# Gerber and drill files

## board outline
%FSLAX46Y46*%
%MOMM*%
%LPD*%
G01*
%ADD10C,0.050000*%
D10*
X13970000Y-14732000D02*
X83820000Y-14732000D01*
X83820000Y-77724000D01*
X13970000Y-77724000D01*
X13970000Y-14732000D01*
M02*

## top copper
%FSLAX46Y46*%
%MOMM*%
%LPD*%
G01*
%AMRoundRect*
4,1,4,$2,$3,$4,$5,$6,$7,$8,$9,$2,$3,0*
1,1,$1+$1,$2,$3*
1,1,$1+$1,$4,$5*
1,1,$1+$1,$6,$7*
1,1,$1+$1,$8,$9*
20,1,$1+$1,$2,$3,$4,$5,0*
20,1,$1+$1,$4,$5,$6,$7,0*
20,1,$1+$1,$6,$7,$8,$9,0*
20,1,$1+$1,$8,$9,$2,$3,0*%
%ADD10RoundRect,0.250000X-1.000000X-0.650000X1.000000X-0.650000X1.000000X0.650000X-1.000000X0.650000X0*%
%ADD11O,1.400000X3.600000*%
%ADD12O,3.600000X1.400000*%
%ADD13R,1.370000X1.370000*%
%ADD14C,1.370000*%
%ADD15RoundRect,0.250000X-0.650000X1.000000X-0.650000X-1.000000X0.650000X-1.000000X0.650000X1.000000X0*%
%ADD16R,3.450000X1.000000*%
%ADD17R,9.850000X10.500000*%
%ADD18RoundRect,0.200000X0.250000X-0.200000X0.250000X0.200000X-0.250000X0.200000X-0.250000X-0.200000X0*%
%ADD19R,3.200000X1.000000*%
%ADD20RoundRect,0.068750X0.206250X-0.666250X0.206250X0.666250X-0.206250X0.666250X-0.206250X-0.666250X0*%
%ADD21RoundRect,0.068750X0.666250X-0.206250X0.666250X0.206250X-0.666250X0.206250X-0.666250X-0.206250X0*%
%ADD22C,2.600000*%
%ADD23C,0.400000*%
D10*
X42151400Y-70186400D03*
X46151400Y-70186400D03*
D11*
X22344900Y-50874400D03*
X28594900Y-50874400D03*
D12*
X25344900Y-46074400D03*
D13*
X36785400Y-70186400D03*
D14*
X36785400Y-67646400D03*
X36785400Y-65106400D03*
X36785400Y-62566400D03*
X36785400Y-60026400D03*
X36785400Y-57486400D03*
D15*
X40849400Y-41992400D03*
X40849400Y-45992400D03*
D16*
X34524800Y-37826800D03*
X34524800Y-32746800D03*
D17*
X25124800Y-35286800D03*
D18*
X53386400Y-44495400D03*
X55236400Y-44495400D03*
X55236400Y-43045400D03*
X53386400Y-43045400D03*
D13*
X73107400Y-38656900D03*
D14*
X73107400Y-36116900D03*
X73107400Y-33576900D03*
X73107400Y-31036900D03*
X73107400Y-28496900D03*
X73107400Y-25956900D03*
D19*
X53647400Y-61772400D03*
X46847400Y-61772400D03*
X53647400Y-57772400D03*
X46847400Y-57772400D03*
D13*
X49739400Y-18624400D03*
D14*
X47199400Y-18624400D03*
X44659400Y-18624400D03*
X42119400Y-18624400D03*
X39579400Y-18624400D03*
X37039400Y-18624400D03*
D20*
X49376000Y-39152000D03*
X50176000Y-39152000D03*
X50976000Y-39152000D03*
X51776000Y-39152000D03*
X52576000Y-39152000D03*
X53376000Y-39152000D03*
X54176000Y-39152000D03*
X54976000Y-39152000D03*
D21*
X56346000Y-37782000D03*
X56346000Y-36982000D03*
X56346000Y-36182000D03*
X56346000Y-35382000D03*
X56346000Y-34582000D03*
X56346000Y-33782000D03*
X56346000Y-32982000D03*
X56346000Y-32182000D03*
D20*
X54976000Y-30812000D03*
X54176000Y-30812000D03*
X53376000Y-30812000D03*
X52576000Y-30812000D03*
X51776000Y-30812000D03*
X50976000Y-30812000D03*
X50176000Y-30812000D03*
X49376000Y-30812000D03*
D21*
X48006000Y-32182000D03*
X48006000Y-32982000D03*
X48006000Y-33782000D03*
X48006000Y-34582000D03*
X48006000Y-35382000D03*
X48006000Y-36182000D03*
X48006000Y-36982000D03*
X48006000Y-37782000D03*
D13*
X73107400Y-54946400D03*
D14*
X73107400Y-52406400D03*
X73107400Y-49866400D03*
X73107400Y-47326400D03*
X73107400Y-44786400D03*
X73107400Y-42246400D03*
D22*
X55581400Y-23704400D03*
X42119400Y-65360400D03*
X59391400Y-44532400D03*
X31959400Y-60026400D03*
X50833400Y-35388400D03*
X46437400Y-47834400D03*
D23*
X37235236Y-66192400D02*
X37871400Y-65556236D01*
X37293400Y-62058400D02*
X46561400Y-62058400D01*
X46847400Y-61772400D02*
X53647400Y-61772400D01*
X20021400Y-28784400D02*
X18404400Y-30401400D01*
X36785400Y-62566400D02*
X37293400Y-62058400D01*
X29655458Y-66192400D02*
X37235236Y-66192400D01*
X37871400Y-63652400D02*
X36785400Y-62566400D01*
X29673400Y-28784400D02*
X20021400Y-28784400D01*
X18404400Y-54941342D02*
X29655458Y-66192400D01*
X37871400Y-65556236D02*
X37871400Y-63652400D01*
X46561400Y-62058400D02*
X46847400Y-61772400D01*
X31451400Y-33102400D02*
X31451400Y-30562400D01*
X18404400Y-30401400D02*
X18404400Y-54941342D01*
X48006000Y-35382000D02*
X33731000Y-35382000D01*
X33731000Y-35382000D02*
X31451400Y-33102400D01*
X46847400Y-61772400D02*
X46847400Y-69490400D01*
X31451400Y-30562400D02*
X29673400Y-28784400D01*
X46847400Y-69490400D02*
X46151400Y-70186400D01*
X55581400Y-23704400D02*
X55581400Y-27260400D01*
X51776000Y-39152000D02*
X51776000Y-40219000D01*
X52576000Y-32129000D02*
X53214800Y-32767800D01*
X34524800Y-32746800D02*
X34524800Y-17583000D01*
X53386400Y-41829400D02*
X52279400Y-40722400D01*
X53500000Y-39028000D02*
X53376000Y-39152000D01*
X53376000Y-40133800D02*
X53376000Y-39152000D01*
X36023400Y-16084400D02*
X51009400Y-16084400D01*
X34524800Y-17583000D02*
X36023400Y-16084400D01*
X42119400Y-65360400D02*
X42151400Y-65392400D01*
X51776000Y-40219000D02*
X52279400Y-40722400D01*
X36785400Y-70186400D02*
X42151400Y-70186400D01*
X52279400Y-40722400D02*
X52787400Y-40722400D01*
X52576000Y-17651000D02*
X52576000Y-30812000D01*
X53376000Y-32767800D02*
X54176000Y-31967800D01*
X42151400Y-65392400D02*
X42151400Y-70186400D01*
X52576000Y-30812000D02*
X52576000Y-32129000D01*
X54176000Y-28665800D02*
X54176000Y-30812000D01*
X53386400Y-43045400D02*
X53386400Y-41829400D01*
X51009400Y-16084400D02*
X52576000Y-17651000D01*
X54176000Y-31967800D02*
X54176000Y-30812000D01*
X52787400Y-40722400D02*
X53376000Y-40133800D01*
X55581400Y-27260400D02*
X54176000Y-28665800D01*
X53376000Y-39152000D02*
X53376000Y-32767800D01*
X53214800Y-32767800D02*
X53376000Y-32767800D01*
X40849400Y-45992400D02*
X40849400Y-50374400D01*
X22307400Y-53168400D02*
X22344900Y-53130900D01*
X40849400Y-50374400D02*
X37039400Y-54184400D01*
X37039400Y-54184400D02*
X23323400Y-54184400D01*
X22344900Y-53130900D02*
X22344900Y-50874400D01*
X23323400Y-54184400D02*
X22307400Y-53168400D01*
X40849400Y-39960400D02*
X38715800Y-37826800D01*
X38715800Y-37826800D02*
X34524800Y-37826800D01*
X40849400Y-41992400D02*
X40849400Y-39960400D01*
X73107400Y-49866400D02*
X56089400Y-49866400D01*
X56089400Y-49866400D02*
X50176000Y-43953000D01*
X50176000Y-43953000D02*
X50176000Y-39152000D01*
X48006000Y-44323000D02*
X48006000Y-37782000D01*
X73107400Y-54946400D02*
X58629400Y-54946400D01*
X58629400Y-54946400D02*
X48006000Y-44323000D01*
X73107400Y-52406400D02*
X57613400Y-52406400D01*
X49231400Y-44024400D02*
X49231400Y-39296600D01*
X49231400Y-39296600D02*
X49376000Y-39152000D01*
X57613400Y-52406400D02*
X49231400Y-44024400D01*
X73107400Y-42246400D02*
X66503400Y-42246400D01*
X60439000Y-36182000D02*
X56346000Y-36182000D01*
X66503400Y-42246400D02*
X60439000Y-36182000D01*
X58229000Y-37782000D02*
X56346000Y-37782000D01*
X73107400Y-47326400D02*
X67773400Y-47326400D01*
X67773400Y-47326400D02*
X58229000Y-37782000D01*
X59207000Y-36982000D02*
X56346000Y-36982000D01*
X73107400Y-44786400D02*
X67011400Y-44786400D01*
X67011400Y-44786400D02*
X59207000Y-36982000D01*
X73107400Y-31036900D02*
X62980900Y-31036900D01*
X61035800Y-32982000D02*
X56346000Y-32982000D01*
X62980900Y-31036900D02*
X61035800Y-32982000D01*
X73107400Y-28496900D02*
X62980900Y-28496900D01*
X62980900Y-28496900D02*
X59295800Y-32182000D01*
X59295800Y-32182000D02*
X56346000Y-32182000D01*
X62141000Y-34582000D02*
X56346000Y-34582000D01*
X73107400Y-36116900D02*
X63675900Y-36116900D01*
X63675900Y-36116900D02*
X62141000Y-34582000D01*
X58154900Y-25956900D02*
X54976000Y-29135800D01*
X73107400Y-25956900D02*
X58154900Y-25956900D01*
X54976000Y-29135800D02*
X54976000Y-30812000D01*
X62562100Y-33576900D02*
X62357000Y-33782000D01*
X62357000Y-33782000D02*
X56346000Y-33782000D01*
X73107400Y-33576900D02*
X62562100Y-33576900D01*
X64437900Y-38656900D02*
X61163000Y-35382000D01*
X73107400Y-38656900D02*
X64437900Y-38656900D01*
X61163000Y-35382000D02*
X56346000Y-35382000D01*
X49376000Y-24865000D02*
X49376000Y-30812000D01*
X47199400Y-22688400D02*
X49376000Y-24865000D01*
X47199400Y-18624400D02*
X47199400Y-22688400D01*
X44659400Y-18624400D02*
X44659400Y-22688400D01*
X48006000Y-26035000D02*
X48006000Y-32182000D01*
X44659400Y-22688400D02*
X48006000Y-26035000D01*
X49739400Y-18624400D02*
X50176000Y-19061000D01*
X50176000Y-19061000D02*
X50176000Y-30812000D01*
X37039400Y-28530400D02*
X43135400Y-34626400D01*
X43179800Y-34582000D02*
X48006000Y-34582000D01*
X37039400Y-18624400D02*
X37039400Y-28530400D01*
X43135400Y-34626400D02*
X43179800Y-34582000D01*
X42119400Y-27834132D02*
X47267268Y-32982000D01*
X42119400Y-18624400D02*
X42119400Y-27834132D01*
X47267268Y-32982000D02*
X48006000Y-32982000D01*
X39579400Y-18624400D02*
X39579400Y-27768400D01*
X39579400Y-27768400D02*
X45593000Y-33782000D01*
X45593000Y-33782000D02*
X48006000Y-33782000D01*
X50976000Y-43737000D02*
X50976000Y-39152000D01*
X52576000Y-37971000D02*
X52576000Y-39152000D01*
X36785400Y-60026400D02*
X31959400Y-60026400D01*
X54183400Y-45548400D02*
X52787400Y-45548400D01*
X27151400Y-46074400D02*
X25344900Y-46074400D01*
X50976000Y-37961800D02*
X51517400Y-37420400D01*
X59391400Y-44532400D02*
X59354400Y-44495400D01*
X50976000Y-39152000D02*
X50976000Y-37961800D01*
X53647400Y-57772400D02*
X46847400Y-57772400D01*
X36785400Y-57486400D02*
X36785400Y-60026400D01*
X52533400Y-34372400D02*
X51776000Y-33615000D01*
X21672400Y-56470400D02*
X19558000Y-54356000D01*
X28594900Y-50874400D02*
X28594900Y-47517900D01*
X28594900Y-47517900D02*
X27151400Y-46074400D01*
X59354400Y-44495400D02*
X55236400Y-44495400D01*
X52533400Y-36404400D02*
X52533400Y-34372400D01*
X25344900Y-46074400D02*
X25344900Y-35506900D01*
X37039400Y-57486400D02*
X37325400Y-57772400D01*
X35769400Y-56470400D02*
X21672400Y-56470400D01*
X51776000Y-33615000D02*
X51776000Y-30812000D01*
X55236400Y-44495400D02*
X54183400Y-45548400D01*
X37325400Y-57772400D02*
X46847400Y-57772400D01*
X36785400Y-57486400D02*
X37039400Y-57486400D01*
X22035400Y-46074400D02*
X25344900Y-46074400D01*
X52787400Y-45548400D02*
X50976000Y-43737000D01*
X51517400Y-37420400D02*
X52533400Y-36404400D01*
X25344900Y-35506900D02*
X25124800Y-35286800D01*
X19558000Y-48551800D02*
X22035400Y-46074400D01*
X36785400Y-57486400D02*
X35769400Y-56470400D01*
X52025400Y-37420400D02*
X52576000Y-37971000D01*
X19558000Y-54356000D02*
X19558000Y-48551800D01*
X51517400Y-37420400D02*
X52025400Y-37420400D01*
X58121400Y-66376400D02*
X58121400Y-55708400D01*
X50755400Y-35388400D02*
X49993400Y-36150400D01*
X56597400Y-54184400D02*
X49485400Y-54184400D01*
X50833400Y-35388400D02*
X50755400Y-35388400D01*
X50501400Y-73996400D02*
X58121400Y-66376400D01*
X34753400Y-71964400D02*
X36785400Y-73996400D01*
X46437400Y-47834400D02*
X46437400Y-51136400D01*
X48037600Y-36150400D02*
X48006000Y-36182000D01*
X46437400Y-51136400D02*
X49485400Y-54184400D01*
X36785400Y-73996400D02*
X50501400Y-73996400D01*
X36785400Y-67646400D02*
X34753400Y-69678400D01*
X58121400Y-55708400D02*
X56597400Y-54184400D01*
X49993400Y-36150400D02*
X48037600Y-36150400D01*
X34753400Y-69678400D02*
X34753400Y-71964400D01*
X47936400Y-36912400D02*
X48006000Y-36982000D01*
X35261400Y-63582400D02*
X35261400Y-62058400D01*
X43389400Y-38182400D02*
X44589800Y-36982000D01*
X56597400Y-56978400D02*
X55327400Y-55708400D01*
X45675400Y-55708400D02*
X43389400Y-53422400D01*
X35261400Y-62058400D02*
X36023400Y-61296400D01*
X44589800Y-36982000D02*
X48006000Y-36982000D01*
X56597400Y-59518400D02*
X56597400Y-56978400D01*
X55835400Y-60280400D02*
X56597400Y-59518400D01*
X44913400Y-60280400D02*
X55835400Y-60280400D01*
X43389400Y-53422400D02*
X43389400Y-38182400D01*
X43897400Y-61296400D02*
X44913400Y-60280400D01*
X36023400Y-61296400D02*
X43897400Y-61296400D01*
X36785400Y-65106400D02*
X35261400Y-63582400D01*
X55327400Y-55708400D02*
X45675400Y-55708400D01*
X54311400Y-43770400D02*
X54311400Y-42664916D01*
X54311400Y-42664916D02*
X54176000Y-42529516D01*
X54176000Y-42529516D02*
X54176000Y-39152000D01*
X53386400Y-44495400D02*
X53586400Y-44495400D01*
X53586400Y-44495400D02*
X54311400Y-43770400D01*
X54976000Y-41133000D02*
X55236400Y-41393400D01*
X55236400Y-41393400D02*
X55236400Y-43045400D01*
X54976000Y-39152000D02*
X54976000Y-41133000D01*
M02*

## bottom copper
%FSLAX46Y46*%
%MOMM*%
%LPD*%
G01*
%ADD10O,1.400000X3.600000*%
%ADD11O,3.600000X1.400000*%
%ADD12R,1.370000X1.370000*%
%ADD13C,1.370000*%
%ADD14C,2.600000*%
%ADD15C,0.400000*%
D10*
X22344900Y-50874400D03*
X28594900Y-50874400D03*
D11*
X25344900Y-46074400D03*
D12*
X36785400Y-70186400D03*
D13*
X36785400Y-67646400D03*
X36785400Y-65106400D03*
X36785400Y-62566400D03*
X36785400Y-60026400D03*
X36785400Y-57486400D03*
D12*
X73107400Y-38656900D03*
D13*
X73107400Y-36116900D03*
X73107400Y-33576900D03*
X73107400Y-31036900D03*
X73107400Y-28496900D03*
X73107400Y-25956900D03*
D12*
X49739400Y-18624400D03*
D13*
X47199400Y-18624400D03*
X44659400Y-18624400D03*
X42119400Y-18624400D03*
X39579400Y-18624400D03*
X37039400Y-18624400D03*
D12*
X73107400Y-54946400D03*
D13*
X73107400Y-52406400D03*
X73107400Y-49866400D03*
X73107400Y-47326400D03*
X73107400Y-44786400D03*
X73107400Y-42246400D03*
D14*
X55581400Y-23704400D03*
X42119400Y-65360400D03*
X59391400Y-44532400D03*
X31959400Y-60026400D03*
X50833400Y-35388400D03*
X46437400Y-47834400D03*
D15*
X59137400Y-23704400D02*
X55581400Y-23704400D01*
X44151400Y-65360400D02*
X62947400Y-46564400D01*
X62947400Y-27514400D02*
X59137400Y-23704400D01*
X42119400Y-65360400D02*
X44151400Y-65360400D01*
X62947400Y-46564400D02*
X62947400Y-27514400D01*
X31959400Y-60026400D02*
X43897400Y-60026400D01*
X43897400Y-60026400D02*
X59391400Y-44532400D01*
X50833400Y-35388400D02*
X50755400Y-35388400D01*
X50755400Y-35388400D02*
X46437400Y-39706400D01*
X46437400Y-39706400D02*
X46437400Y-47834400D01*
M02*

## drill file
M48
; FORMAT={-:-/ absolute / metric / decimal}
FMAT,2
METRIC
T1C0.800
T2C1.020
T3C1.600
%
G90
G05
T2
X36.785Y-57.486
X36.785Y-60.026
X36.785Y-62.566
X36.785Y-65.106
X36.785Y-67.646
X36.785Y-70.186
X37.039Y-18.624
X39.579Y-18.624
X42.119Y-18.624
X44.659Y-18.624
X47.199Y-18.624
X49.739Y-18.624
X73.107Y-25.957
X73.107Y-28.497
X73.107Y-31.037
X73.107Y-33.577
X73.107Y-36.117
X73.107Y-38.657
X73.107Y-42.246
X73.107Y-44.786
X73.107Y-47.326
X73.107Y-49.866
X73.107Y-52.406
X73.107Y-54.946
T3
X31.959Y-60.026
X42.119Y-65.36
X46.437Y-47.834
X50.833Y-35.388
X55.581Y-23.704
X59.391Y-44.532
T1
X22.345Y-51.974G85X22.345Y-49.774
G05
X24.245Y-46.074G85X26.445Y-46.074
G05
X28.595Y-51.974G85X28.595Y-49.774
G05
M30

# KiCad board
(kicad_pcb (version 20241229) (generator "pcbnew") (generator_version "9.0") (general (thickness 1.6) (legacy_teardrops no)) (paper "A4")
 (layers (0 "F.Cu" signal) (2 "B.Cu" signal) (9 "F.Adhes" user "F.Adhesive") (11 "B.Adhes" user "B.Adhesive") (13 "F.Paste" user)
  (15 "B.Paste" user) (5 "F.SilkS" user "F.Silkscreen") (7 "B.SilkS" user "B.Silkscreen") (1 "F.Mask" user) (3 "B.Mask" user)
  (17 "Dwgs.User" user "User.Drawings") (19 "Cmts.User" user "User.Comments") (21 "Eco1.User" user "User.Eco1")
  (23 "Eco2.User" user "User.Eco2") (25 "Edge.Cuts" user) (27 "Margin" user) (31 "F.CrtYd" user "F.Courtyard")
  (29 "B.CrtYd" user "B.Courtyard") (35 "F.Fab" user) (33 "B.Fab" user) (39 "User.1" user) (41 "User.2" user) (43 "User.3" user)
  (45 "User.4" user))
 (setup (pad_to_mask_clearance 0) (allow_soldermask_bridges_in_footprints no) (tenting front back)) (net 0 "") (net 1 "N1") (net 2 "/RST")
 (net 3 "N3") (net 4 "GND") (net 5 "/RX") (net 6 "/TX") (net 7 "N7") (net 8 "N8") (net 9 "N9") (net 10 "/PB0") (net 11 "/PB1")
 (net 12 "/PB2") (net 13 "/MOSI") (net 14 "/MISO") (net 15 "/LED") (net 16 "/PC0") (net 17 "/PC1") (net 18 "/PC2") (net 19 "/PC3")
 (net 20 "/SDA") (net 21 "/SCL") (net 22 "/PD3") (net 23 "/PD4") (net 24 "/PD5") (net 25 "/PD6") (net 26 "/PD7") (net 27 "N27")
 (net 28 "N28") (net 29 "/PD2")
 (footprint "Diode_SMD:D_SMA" (layer "F.Cu") (at 44.1514 70.1864)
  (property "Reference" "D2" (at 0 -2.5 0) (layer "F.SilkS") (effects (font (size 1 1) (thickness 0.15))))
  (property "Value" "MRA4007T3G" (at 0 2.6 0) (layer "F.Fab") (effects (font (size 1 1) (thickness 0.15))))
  (pad "1" smd roundrect (at -2 0) (size 2.5 1.8) (layers "F.Cu" "F.Mask" "F.Paste") (roundrect_rratio 0.1388888889) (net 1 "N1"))
  (pad "2" smd roundrect (at 2 0) (size 2.5 1.8) (layers "F.Cu" "F.Mask" "F.Paste") (roundrect_rratio 0.1388888889) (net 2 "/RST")))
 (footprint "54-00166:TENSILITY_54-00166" (layer "F.Cu") (at 28.5949 50.8744 90)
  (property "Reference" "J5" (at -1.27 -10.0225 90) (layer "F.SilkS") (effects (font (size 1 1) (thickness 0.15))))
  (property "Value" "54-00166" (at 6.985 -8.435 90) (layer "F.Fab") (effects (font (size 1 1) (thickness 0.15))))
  (pad "A" thru_hole oval (at 0 -6.25 90) (size 3.6 1.4) (drill oval 3 0.8) (layers "*.Cu" "*.Mask") (remove_unused_layers no) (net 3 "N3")
   (solder_mask_margin 0.102))
  (pad "B" thru_hole oval (at 0 0 90) (size 3.6 1.4) (drill oval 3 0.8) (layers "*.Cu" "*.Mask") (remove_unused_layers no) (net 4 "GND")
   (solder_mask_margin 0.102))
  (pad "C" thru_hole oval (at 4.8 -3.25 90) (size 1.4 3.6) (drill oval 0.8 3) (layers "*.Cu" "*.Mask") (remove_unused_layers no)
   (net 4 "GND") (solder_mask_margin 0.102)))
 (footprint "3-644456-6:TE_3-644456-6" (layer "F.Cu") (at 36.7854 70.1864 90)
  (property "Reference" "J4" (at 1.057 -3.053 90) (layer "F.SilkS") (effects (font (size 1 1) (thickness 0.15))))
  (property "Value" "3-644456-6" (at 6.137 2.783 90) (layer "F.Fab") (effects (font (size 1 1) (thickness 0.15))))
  (pad "1" thru_hole rect (at 0 0 90) (size 1.37 1.37) (drill 1.02) (layers "*.Cu" "*.Mask") (remove_unused_layers no) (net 1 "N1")
   (solder_mask_margin 0.102))
  (pad "2" thru_hole circle (at 2.54 0 90) (size 1.37 1.37) (drill 1.02) (layers "*.Cu" "*.Mask") (remove_unused_layers no) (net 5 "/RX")
   (solder_mask_margin 0.102))
  (pad "3" thru_hole circle (at 5.08 0 90) (size 1.37 1.37) (drill 1.02) (layers "*.Cu" "*.Mask") (remove_unused_layers no) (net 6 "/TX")
   (solder_mask_margin 0.102))
  (pad "4" thru_hole circle (at 7.62 0 90) (size 1.37 1.37) (drill 1.02) (layers "*.Cu" "*.Mask") (remove_unused_layers no) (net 2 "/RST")
   (solder_mask_margin 0.102))
  (pad "5" thru_hole circle (at 10.16 0 90) (size 1.37 1.37) (drill 1.02) (layers "*.Cu" "*.Mask") (remove_unused_layers no) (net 4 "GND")
   (solder_mask_margin 0.102))
  (pad "6" thru_hole circle (at 12.7 0 90) (size 1.37 1.37) (drill 1.02) (layers "*.Cu" "*.Mask") (remove_unused_layers no) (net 4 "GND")
   (solder_mask_margin 0.102)))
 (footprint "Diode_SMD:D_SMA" (layer "F.Cu") (at 40.8494 43.9924 -90)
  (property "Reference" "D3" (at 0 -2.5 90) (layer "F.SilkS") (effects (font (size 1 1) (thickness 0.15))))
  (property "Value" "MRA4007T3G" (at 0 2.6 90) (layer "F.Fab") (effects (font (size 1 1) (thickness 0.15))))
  (pad "1" smd roundrect (at -2 0 270) (size 2.5 1.8) (layers "F.Cu" "F.Mask" "F.Paste") (roundrect_rratio 0.1388888889) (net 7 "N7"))
  (pad "2" smd roundrect (at 2 0 270) (size 2.5 1.8) (layers "F.Cu" "F.Mask" "F.Paste") (roundrect_rratio 0.1388888889) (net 3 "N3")))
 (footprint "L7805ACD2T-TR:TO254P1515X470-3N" (layer "F.Cu") (at 28.2248 35.2868 180)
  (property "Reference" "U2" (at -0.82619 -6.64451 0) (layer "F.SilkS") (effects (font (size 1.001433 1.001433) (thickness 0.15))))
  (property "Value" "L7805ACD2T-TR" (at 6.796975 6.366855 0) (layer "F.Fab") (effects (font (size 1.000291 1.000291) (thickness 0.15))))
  (pad "1" smd rect (at -6.3 -2.54 180) (size 3.45 1) (layers "F.Cu" "F.Mask" "F.Paste") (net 7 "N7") (solder_mask_margin 0.102))
  (pad "2" smd rect (at -6.3 2.54 180) (size 3.45 1) (layers "F.Cu" "F.Mask" "F.Paste") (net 1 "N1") (solder_mask_margin 0.102))
  (pad "3" smd rect (at 3.1 0 180) (size 9.85 10.5) (layers "F.Cu" "F.Mask") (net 4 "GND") (solder_mask_margin 0.102)))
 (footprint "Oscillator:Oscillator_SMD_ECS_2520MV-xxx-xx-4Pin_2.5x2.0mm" (layer "F.Cu") (at 54.3114 43.7704 90)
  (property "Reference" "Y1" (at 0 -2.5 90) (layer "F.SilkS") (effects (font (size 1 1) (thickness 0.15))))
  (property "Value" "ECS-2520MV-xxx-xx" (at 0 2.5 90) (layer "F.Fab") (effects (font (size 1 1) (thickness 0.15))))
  (pad "1" smd roundrect (at -0.725 -0.925 90) (size 0.8 0.9) (layers "F.Cu" "F.Mask" "F.Paste") (roundrect_rratio 0.25) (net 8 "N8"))
  (pad "2" smd roundrect (at -0.725 0.925 90) (size 0.8 0.9) (layers "F.Cu" "F.Mask" "F.Paste") (roundrect_rratio 0.25) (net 4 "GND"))
  (pad "3" smd roundrect (at 0.725 0.925 90) (size 0.8 0.9) (layers "F.Cu" "F.Mask" "F.Paste") (roundrect_rratio 0.25) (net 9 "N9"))
  (pad "4" smd roundrect (at 0.725 -0.925 90) (size 0.8 0.9) (layers "F.Cu" "F.Mask" "F.Paste") (roundrect_rratio 0.25) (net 1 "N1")))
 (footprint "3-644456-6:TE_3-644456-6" (layer "F.Cu") (at 73.1074 38.6569 90)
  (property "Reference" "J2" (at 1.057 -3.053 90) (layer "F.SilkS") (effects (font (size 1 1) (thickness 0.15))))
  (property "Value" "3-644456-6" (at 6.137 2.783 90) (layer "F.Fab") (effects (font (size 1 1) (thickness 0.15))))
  (pad "1" thru_hole rect (at 0 0 90) (size 1.37 1.37) (drill 1.02) (layers "*.Cu" "*.Mask") (remove_unused_layers no) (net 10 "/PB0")
   (solder_mask_margin 0.102))
  (pad "2" thru_hole circle (at 2.54 0 90) (size 1.37 1.37) (drill 1.02) (layers "*.Cu" "*.Mask") (remove_unused_layers no) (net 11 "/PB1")
   (solder_mask_margin 0.102))
  (pad "3" thru_hole circle (at 5.08 0 90) (size 1.37 1.37) (drill 1.02) (layers "*.Cu" "*.Mask") (remove_unused_layers no) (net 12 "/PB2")
   (solder_mask_margin 0.102))
  (pad "4" thru_hole circle (at 7.62 0 90) (size 1.37 1.37) (drill 1.02) (layers "*.Cu" "*.Mask") (remove_unused_layers no) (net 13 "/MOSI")
   (solder_mask_margin 0.102))
  (pad "5" thru_hole circle (at 10.16 0 90) (size 1.37 1.37) (drill 1.02) (layers "*.Cu" "*.Mask") (remove_unused_layers no)
   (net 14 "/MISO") (solder_mask_margin 0.102))
  (pad "6" thru_hole circle (at 12.7 0 90) (size 1.37 1.37) (drill 1.02) (layers "*.Cu" "*.Mask") (remove_unused_layers no) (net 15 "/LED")
   (solder_mask_margin 0.102)))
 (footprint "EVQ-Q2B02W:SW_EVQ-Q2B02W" (layer "F.Cu") (at 50.2474 59.7724)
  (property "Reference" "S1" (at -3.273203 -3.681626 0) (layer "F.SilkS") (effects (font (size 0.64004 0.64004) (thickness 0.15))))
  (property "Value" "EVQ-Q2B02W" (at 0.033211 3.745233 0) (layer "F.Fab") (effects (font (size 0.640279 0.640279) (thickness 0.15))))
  (pad "A" smd rect (at 3.4 2) (size 3.2 1) (layers "F.Cu" "F.Mask" "F.Paste") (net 2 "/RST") (solder_mask_margin 0.102))
  (pad "A'" smd rect (at -3.4 2) (size 3.2 1) (layers "F.Cu" "F.Mask" "F.Paste") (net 2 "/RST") (solder_mask_margin 0.102))
  (pad "B" smd rect (at 3.4 -2) (size 3.2 1) (layers "F.Cu" "F.Mask" "F.Paste") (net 4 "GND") (solder_mask_margin 0.102))
  (pad "B'" smd rect (at -3.4 -2) (size 3.2 1) (layers "F.Cu" "F.Mask" "F.Paste") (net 4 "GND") (solder_mask_margin 0.102)))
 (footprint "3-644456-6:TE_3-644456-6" (layer "F.Cu") (at 49.7394 18.6244 180)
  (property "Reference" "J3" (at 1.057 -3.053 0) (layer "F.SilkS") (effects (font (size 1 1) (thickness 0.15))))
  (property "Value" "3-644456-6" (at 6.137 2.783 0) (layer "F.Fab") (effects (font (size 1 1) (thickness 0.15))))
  (pad "1" thru_hole rect (at 0 0 180) (size 1.37 1.37) (drill 1.02) (layers "*.Cu" "*.Mask") (remove_unused_layers no) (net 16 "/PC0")
   (solder_mask_margin 0.102))
  (pad "2" thru_hole circle (at 2.54 0 180) (size 1.37 1.37) (drill 1.02) (layers "*.Cu" "*.Mask") (remove_unused_layers no) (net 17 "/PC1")
   (solder_mask_margin 0.102))
  (pad "3" thru_hole circle (at 5.08 0 180) (size 1.37 1.37) (drill 1.02) (layers "*.Cu" "*.Mask") (remove_unused_layers no) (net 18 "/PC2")
   (solder_mask_margin 0.102))
  (pad "4" thru_hole circle (at 7.62 0 180) (size 1.37 1.37) (drill 1.02) (layers "*.Cu" "*.Mask") (remove_unused_layers no) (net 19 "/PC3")
   (solder_mask_margin 0.102))
  (pad "5" thru_hole circle (at 10.16 0 180) (size 1.37 1.37) (drill 1.02) (layers "*.Cu" "*.Mask") (remove_unused_layers no)
   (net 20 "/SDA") (solder_mask_margin 0.102))
  (pad "6" thru_hole circle (at 12.7 0 180) (size 1.37 1.37) (drill 1.02) (layers "*.Cu" "*.Mask") (remove_unused_layers no) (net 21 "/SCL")
   (solder_mask_margin 0.102)))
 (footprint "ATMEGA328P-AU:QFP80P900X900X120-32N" (layer "F.Cu") (at 52.176 34.982 90)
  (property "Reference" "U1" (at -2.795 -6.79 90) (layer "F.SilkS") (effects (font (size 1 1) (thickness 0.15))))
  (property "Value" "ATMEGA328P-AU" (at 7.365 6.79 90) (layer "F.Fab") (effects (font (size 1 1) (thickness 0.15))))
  (pad "1" smd roundrect (at -4.17 -2.8 90) (size 1.47 0.55) (layers "F.Cu" "F.Mask" "F.Paste") (roundrect_rratio 0.125) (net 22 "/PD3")
   (solder_mask_margin 0.102))
  (pad "2" smd roundrect (at -4.17 -2 90) (size 1.47 0.55) (layers "F.Cu" "F.Mask" "F.Paste") (roundrect_rratio 0.125) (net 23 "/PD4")
   (solder_mask_margin 0.102))
  (pad "3" smd roundrect (at -4.17 -1.2 90) (size 1.47 0.55) (layers "F.Cu" "F.Mask" "F.Paste") (roundrect_rratio 0.125) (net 4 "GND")
   (solder_mask_margin 0.102))
  (pad "4" smd roundrect (at -4.17 -0.4 90) (size 1.47 0.55) (layers "F.Cu" "F.Mask" "F.Paste") (roundrect_rratio 0.125) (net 1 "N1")
   (solder_mask_margin 0.102))
  (pad "5" smd roundrect (at -4.17 0.4 90) (size 1.47 0.55) (layers "F.Cu" "F.Mask" "F.Paste") (roundrect_rratio 0.125) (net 4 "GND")
   (solder_mask_margin 0.102))
  (pad "6" smd roundrect (at -4.17 1.2 90) (size 1.47 0.55) (layers "F.Cu" "F.Mask" "F.Paste") (roundrect_rratio 0.125) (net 1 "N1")
   (solder_mask_margin 0.102))
  (pad "7" smd roundrect (at -4.17 2 90) (size 1.47 0.55) (layers "F.Cu" "F.Mask" "F.Paste") (roundrect_rratio 0.125) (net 8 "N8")
   (solder_mask_margin 0.102))
  (pad "8" smd roundrect (at -4.17 2.8 90) (size 1.47 0.55) (layers "F.Cu" "F.Mask" "F.Paste") (roundrect_rratio 0.125) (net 9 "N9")
   (solder_mask_margin 0.102))
  (pad "9" smd roundrect (at -2.8 4.17 90) (size 0.55 1.47) (layers "F.Cu" "F.Mask" "F.Paste") (roundrect_rratio 0.125) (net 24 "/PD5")
   (solder_mask_margin 0.102))
  (pad "10" smd roundrect (at -2 4.17 90) (size 0.55 1.47) (layers "F.Cu" "F.Mask" "F.Paste") (roundrect_rratio 0.125) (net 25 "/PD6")
   (solder_mask_margin 0.102))
  (pad "11" smd roundrect (at -1.2 4.17 90) (size 0.55 1.47) (layers "F.Cu" "F.Mask" "F.Paste") (roundrect_rratio 0.125) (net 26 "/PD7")
   (solder_mask_margin 0.102))
  (pad "12" smd roundrect (at -0.4 4.17 90) (size 0.55 1.47) (layers "F.Cu" "F.Mask" "F.Paste") (roundrect_rratio 0.125) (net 10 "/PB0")
   (solder_mask_margin 0.102))
  (pad "13" smd roundrect (at 0.4 4.17 90) (size 0.55 1.47) (layers "F.Cu" "F.Mask" "F.Paste") (roundrect_rratio 0.125) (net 11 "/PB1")
   (solder_mask_margin 0.102))
  (pad "14" smd roundrect (at 1.2 4.17 90) (size 0.55 1.47) (layers "F.Cu" "F.Mask" "F.Paste") (roundrect_rratio 0.125) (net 12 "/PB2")
   (solder_mask_margin 0.102))
  (pad "15" smd roundrect (at 2 4.17 90) (size 0.55 1.47) (layers "F.Cu" "F.Mask" "F.Paste") (roundrect_rratio 0.125) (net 13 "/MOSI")
   (solder_mask_margin 0.102))
  (pad "16" smd roundrect (at 2.8 4.17 90) (size 0.55 1.47) (layers "F.Cu" "F.Mask" "F.Paste") (roundrect_rratio 0.125) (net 14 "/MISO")
   (solder_mask_margin 0.102))
  (pad "17" smd roundrect (at 4.17 2.8 90) (size 1.47 0.55) (layers "F.Cu" "F.Mask" "F.Paste") (roundrect_rratio 0.125) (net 15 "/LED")
   (solder_mask_margin 0.102))
  (pad "18" smd roundrect (at 4.17 2 90) (size 1.47 0.55) (layers "F.Cu" "F.Mask" "F.Paste") (roundrect_rratio 0.125) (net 1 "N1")
   (solder_mask_margin 0.102))
  (pad "19" smd roundrect (at 4.17 1.2 90) (size 1.47 0.55) (layers "F.Cu" "F.Mask" "F.Paste") (roundrect_rratio 0.125) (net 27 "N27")
   (solder_mask_margin 0.102))
  (pad "20" smd roundrect (at 4.17 0.4 90) (size 1.47 0.55) (layers "F.Cu" "F.Mask" "F.Paste") (roundrect_rratio 0.125) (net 1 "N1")
   (solder_mask_margin 0.102))
  (pad "21" smd roundrect (at 4.17 -0.4 90) (size 1.47 0.55) (layers "F.Cu" "F.Mask" "F.Paste") (roundrect_rratio 0.125) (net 4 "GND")
   (solder_mask_margin 0.102))
  (pad "22" smd roundrect (at 4.17 -1.2 90) (size 1.47 0.55) (layers "F.Cu" "F.Mask" "F.Paste") (roundrect_rratio 0.125) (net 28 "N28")
   (solder_mask_margin 0.102))
  (pad "23" smd roundrect (at 4.17 -2 90) (size 1.47 0.55) (layers "F.Cu" "F.Mask" "F.Paste") (roundrect_rratio 0.125) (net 16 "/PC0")
   (solder_mask_margin 0.102))
  (pad "24" smd roundrect (at 4.17 -2.8 90) (size 1.47 0.55) (layers "F.Cu" "F.Mask" "F.Paste") (roundrect_rratio 0.125) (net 17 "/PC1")
   (solder_mask_margin 0.102))
  (pad "25" smd roundrect (at 2.8 -4.17 90) (size 0.55 1.47) (layers "F.Cu" "F.Mask" "F.Paste") (roundrect_rratio 0.125) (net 18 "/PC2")
   (solder_mask_margin 0.102))
  (pad "26" smd roundrect (at 2 -4.17 90) (size 0.55 1.47) (layers "F.Cu" "F.Mask" "F.Paste") (roundrect_rratio 0.125) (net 19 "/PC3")
   (solder_mask_margin 0.102))
  (pad "27" smd roundrect (at 1.2 -4.17 90) (size 0.55 1.47) (layers "F.Cu" "F.Mask" "F.Paste") (roundrect_rratio 0.125) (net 20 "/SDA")
   (solder_mask_margin 0.102))
  (pad "28" smd roundrect (at 0.4 -4.17 90) (size 0.55 1.47) (layers "F.Cu" "F.Mask" "F.Paste") (roundrect_rratio 0.125) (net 21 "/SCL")
   (solder_mask_margin 0.102))
  (pad "29" smd roundrect (at -0.4 -4.17 90) (size 0.55 1.47) (layers "F.Cu" "F.Mask" "F.Paste") (roundrect_rratio 0.125) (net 2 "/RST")
   (solder_mask_margin 0.102))
  (pad "30" smd roundrect (at -1.2 -4.17 90) (size 0.55 1.47) (layers "F.Cu" "F.Mask" "F.Paste") (roundrect_rratio 0.125) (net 5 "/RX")
   (solder_mask_margin 0.102))
  (pad "31" smd roundrect (at -2 -4.17 90) (size 0.55 1.47) (layers "F.Cu" "F.Mask" "F.Paste") (roundrect_rratio 0.125) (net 6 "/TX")
   (solder_mask_margin 0.102))
  (pad "32" smd roundrect (at -2.8 -4.17 90) (size 0.55 1.47) (layers "F.Cu" "F.Mask" "F.Paste") (roundrect_rratio 0.125) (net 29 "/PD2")
   (solder_mask_margin 0.102)))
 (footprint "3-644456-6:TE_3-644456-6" (layer "F.Cu") (at 73.1074 54.9464 90)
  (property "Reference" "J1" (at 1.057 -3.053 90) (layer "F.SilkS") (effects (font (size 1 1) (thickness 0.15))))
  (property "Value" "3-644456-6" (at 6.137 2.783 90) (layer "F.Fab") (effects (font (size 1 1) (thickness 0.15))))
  (pad "1" thru_hole rect (at 0 0 90) (size 1.37 1.37) (drill 1.02) (layers "*.Cu" "*.Mask") (remove_unused_layers no) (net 29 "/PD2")
   (solder_mask_margin 0.102))
  (pad "2" thru_hole circle (at 2.54 0 90) (size 1.37 1.37) (drill 1.02) (layers "*.Cu" "*.Mask") (remove_unused_layers no) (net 22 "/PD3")
   (solder_mask_margin 0.102))
  (pad "3" thru_hole circle (at 5.08 0 90) (size 1.37 1.37) (drill 1.02) (layers "*.Cu" "*.Mask") (remove_unused_layers no) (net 23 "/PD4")
   (solder_mask_margin 0.102))
  (pad "4" thru_hole circle (at 7.62 0 90) (size 1.37 1.37) (drill 1.02) (layers "*.Cu" "*.Mask") (remove_unused_layers no) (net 24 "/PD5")
   (solder_mask_margin 0.102))
  (pad "5" thru_hole circle (at 10.16 0 90) (size 1.37 1.37) (drill 1.02) (layers "*.Cu" "*.Mask") (remove_unused_layers no) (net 25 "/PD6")
   (solder_mask_margin 0.102))
  (pad "6" thru_hole circle (at 12.7 0 90) (size 1.37 1.37) (drill 1.02) (layers "*.Cu" "*.Mask") (remove_unused_layers no) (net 26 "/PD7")
   (solder_mask_margin 0.102)))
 (gr_rect (start 13.97 14.732) (end 83.82 77.724) (stroke (width 0.05) (type default)) (fill no) (layer "Edge.Cuts"))
 (segment (start 37.235236 66.1924) (end 37.8714 65.556236) (width 0.4) (layer "F.Cu") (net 2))
 (segment (start 37.2934 62.0584) (end 46.5614 62.0584) (width 0.4) (layer "F.Cu") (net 2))
 (segment (start 46.8474 61.7724) (end 53.6474 61.7724) (width 0.4) (layer "F.Cu") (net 2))
 (segment (start 20.0214 28.7844) (end 18.4044 30.4014) (width 0.4) (layer "F.Cu") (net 2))
 (segment (start 36.7854 62.5664) (end 37.2934 62.0584) (width 0.4) (layer "F.Cu") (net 2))
 (segment (start 29.655458 66.1924) (end 37.235236 66.1924) (width 0.4) (layer "F.Cu") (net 2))
 (segment (start 37.8714 63.6524) (end 36.7854 62.5664) (width 0.4) (layer "F.Cu") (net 2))
 (segment (start 29.6734 28.7844) (end 20.0214 28.7844) (width 0.4) (layer "F.Cu") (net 2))
 (segment (start 18.4044 54.941342) (end 29.655458 66.1924) (width 0.4) (layer "F.Cu") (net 2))
 (segment (start 37.8714 65.556236) (end 37.8714 63.6524) (width 0.4) (layer "F.Cu") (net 2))
 (segment (start 46.5614 62.0584) (end 46.8474 61.7724) (width 0.4) (layer "F.Cu") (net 2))
 (segment (start 31.4514 33.1024) (end 31.4514 30.5624) (width 0.4) (layer "F.Cu") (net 2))
 (segment (start 18.4044 30.4014) (end 18.4044 54.941342) (width 0.4) (layer "F.Cu") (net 2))
 (segment (start 48.006 35.382) (end 33.731 35.382) (width 0.4) (layer "F.Cu") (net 2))
 (segment (start 33.731 35.382) (end 31.4514 33.1024) (width 0.4) (layer "F.Cu") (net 2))
 (segment (start 46.8474 61.7724) (end 46.8474 69.4904) (width 0.4) (layer "F.Cu") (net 2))
 (segment (start 31.4514 30.5624) (end 29.6734 28.7844) (width 0.4) (layer "F.Cu") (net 2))
 (segment (start 46.8474 69.4904) (end 46.1514 70.1864) (width 0.4) (layer "F.Cu") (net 2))
 (segment (start 55.5814 23.7044) (end 55.5814 27.2604) (width 0.4) (layer "F.Cu") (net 1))
 (segment (start 51.776 39.152) (end 51.776 40.219) (width 0.4) (layer "F.Cu") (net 1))
 (segment (start 52.576 32.129) (end 53.2148 32.7678) (width 0.4) (layer "F.Cu") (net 1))
 (segment (start 34.5248 32.7468) (end 34.5248 17.583) (width 0.4) (layer "F.Cu") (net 1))
 (segment (start 53.3864 41.8294) (end 52.2794 40.7224) (width 0.4) (layer "F.Cu") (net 1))
 (segment (start 53.5 39.028) (end 53.376 39.152) (width 0.4) (layer "F.Cu") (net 1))
 (segment (start 53.376 40.1338) (end 53.376 39.152) (width 0.4) (layer "F.Cu") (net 1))
 (segment (start 36.0234 16.0844) (end 51.0094 16.0844) (width 0.4) (layer "F.Cu") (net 1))
 (segment (start 34.5248 17.583) (end 36.0234 16.0844) (width 0.4) (layer "F.Cu") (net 1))
 (segment (start 42.1194 65.3604) (end 42.1514 65.3924) (width 0.4) (layer "F.Cu") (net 1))
 (segment (start 51.776 40.219) (end 52.2794 40.7224) (width 0.4) (layer "F.Cu") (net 1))
 (segment (start 36.7854 70.1864) (end 42.1514 70.1864) (width 0.4) (layer "F.Cu") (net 1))
 (segment (start 52.2794 40.7224) (end 52.7874 40.7224) (width 0.4) (layer "F.Cu") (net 1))
 (segment (start 52.576 17.651) (end 52.576 30.812) (width 0.4) (layer "F.Cu") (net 1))
 (segment (start 53.376 32.7678) (end 54.176 31.9678) (width 0.4) (layer "F.Cu") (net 1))
 (segment (start 42.1514 65.3924) (end 42.1514 70.1864) (width 0.4) (layer "F.Cu") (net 1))
 (segment (start 52.576 30.812) (end 52.576 32.129) (width 0.4) (layer "F.Cu") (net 1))
 (segment (start 54.176 28.6658) (end 54.176 30.812) (width 0.4) (layer "F.Cu") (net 1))
 (segment (start 53.3864 43.0454) (end 53.3864 41.8294) (width 0.4) (layer "F.Cu") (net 1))
 (segment (start 51.0094 16.0844) (end 52.576 17.651) (width 0.4) (layer "F.Cu") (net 1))
 (segment (start 54.176 31.9678) (end 54.176 30.812) (width 0.4) (layer "F.Cu") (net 1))
 (segment (start 52.7874 40.7224) (end 53.376 40.1338) (width 0.4) (layer "F.Cu") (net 1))
 (segment (start 55.5814 27.2604) (end 54.176 28.6658) (width 0.4) (layer "F.Cu") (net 1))
 (segment (start 53.376 39.152) (end 53.376 32.7678) (width 0.4) (layer "F.Cu") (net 1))
 (segment (start 53.2148 32.7678) (end 53.376 32.7678) (width 0.4) (layer "F.Cu") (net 1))
 (via (at 55.5814 23.7044) (size 2.6) (drill 1.6) (layers "F.Cu" "B.Cu") (free yes) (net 1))
 (via (at 42.1194 65.3604) (size 2.6) (drill 1.6) (layers "F.Cu" "B.Cu") (free yes) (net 1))
 (segment (start 59.1374 23.7044) (end 55.5814 23.7044) (width 0.4) (layer "B.Cu") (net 1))
 (segment (start 44.1514 65.3604) (end 62.9474 46.5644) (width 0.4) (layer "B.Cu") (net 1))
 (segment (start 62.9474 27.5144) (end 59.1374 23.7044) (width 0.4) (layer "B.Cu") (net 1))
 (segment (start 42.1194 65.3604) (end 44.1514 65.3604) (width 0.4) (layer "B.Cu") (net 1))
 (segment (start 62.9474 46.5644) (end 62.9474 27.5144) (width 0.4) (layer "B.Cu") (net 1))
 (segment (start 40.8494 45.9924) (end 40.8494 50.3744) (width 0.4) (layer "F.Cu") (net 3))
 (segment (start 22.3074 53.1684) (end 22.3449 53.1309) (width 0.4) (layer "F.Cu") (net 3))
 (segment (start 40.8494 50.3744) (end 37.0394 54.1844) (width 0.4) (layer "F.Cu") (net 3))
 (segment (start 37.0394 54.1844) (end 23.3234 54.1844) (width 0.4) (layer "F.Cu") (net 3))
 (segment (start 22.3449 53.1309) (end 22.3449 50.8744) (width 0.4) (layer "F.Cu") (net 3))
 (segment (start 23.3234 54.1844) (end 22.3074 53.1684) (width 0.4) (layer "F.Cu") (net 3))
 (segment (start 40.8494 39.9604) (end 38.7158 37.8268) (width 0.4) (layer "F.Cu") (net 7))
 (segment (start 38.7158 37.8268) (end 34.5248 37.8268) (width 0.4) (layer "F.Cu") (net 7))
 (segment (start 40.8494 41.9924) (end 40.8494 39.9604) (width 0.4) (layer "F.Cu") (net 7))
 (segment (start 73.1074 49.8664) (end 56.0894 49.8664) (width 0.4) (layer "F.Cu") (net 23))
 (segment (start 56.0894 49.8664) (end 50.176 43.953) (width 0.4) (layer "F.Cu") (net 23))
 (segment (start 50.176 43.953) (end 50.176 39.152) (width 0.4) (layer "F.Cu") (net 23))
 (segment (start 48.006 44.323) (end 48.006 37.782) (width 0.4) (layer "F.Cu") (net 29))
 (segment (start 73.1074 54.9464) (end 58.6294 54.9464) (width 0.4) (layer "F.Cu") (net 29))
 (segment (start 58.6294 54.9464) (end 48.006 44.323) (width 0.4) (layer "F.Cu") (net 29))
 (segment (start 73.1074 52.4064) (end 57.6134 52.4064) (width 0.4) (layer "F.Cu") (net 22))
 (segment (start 49.2314 44.0244) (end 49.2314 39.2966) (width 0.4) (layer "F.Cu") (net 22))
 (segment (start 49.2314 39.2966) (end 49.376 39.152) (width 0.4) (layer "F.Cu") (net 22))
 (segment (start 57.6134 52.4064) (end 49.2314 44.0244) (width 0.4) (layer "F.Cu") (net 22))
 (segment (start 73.1074 42.2464) (end 66.5034 42.2464) (width 0.4) (layer "F.Cu") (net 26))
 (segment (start 60.439 36.182) (end 56.346 36.182) (width 0.4) (layer "F.Cu") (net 26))
 (segment (start 66.5034 42.2464) (end 60.439 36.182) (width 0.4) (layer "F.Cu") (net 26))
 (segment (start 58.229 37.782) (end 56.346 37.782) (width 0.4) (layer "F.Cu") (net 24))
 (segment (start 73.1074 47.3264) (end 67.7734 47.3264) (width 0.4) (layer "F.Cu") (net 24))
 (segment (start 67.7734 47.3264) (end 58.229 37.782) (width 0.4) (layer "F.Cu") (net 24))
 (segment (start 59.207 36.982) (end 56.346 36.982) (width 0.4) (layer "F.Cu") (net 25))
 (segment (start 73.1074 44.7864) (end 67.0114 44.7864) (width 0.4) (layer "F.Cu") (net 25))
 (segment (start 67.0114 44.7864) (end 59.207 36.982) (width 0.4) (layer "F.Cu") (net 25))
 (segment (start 73.1074 31.0369) (end 62.9809 31.0369) (width 0.4) (layer "F.Cu") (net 13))
 (segment (start 61.0358 32.982) (end 56.346 32.982) (width 0.4) (layer "F.Cu") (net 13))
 (segment (start 62.9809 31.0369) (end 61.0358 32.982) (width 0.4) (layer "F.Cu") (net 13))
 (segment (start 73.1074 28.4969) (end 62.9809 28.4969) (width 0.4) (layer "F.Cu") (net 14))
 (segment (start 62.9809 28.4969) (end 59.2958 32.182) (width 0.4) (layer "F.Cu") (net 14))
 (segment (start 59.2958 32.182) (end 56.346 32.182) (width 0.4) (layer "F.Cu") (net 14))
 (segment (start 62.141 34.582) (end 56.346 34.582) (width 0.4) (layer "F.Cu") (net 11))
 (segment (start 73.1074 36.1169) (end 63.6759 36.1169) (width 0.4) (layer "F.Cu") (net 11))
 (segment (start 63.6759 36.1169) (end 62.141 34.582) (width 0.4) (layer "F.Cu") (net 11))
 (segment (start 58.1549 25.9569) (end 54.976 29.1358) (width 0.4) (layer "F.Cu") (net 15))
 (segment (start 73.1074 25.9569) (end 58.1549 25.9569) (width 0.4) (layer "F.Cu") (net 15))
 (segment (start 54.976 29.1358) (end 54.976 30.812) (width 0.4) (layer "F.Cu") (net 15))
 (segment (start 62.5621 33.5769) (end 62.357 33.782) (width 0.4) (layer "F.Cu") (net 12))
 (segment (start 62.357 33.782) (end 56.346 33.782) (width 0.4) (layer "F.Cu") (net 12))
 (segment (start 73.1074 33.5769) (end 62.5621 33.5769) (width 0.4) (layer "F.Cu") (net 12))
 (segment (start 64.4379 38.6569) (end 61.163 35.382) (width 0.4) (layer "F.Cu") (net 10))
 (segment (start 73.1074 38.6569) (end 64.4379 38.6569) (width 0.4) (layer "F.Cu") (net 10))
 (segment (start 61.163 35.382) (end 56.346 35.382) (width 0.4) (layer "F.Cu") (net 10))
 (segment (start 49.376 24.865) (end 49.376 30.812) (width 0.4) (layer "F.Cu") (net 17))
 (segment (start 47.1994 22.6884) (end 49.376 24.865) (width 0.4) (layer "F.Cu") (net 17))
 (segment (start 47.1994 18.6244) (end 47.1994 22.6884) (width 0.4) (layer "F.Cu") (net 17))
 (segment (start 44.6594 18.6244) (end 44.6594 22.6884) (width 0.4) (layer "F.Cu") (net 18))
 (segment (start 48.006 26.035) (end 48.006 32.182) (width 0.4) (layer "F.Cu") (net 18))
 (segment (start 44.6594 22.6884) (end 48.006 26.035) (width 0.4) (layer "F.Cu") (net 18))
 (segment (start 49.7394 18.6244) (end 50.176 19.061) (width 0.4) (layer "F.Cu") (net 16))
 (segment (start 50.176 19.061) (end 50.176 30.812) (width 0.4) (layer "F.Cu") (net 16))
 (segment (start 37.0394 28.5304) (end 43.1354 34.6264) (width 0.4) (layer "F.Cu") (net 21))
 (segment (start 43.1798 34.582) (end 48.006 34.582) (width 0.4) (layer "F.Cu") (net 21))
 (segment (start 37.0394 18.6244) (end 37.0394 28.5304) (width 0.4) (layer "F.Cu") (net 21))
 (segment (start 43.1354 34.6264) (end 43.1798 34.582) (width 0.4) (layer "F.Cu") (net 21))
 (segment (start 42.1194 27.834132) (end 47.267268 32.982) (width 0.4) (layer "F.Cu") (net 19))
 (segment (start 42.1194 18.6244) (end 42.1194 27.834132) (width 0.4) (layer "F.Cu") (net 19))
 (segment (start 47.267268 32.982) (end 48.006 32.982) (width 0.4) (layer "F.Cu") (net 19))
 (segment (start 39.5794 18.6244) (end 39.5794 27.7684) (width 0.4) (layer "F.Cu") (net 20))
 (segment (start 39.5794 27.7684) (end 45.593 33.782) (width 0.4) (layer "F.Cu") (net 20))
 (segment (start 45.593 33.782) (end 48.006 33.782) (width 0.4) (layer "F.Cu") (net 20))
 (segment (start 50.976 43.737) (end 50.976 39.152) (width 0.4) (layer "F.Cu") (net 4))
 (segment (start 52.576 37.971) (end 52.576 39.152) (width 0.4) (layer "F.Cu") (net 4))
 (segment (start 36.7854 60.0264) (end 31.9594 60.0264) (width 0.4) (layer "F.Cu") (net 4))
 (segment (start 54.1834 45.5484) (end 52.7874 45.5484) (width 0.4) (layer "F.Cu") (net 4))
 (segment (start 27.1514 46.0744) (end 25.3449 46.0744) (width 0.4) (layer "F.Cu") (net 4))
 (segment (start 50.976 37.9618) (end 51.5174 37.4204) (width 0.4) (layer "F.Cu") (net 4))
 (segment (start 59.3914 44.5324) (end 59.3544 44.4954) (width 0.4) (layer "F.Cu") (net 4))
 (segment (start 50.976 39.152) (end 50.976 37.9618) (width 0.4) (layer "F.Cu") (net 4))
 (segment (start 53.6474 57.7724) (end 46.8474 57.7724) (width 0.4) (layer "F.Cu") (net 4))
 (segment (start 36.7854 57.4864) (end 36.7854 60.0264) (width 0.4) (layer "F.Cu") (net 4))
 (segment (start 52.5334 34.3724) (end 51.776 33.615) (width 0.4) (layer "F.Cu") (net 4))
 (segment (start 21.6724 56.4704) (end 19.558 54.356) (width 0.4) (layer "F.Cu") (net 4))
 (segment (start 28.5949 50.8744) (end 28.5949 47.5179) (width 0.4) (layer "F.Cu") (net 4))
 (segment (start 28.5949 47.5179) (end 27.1514 46.0744) (width 0.4) (layer "F.Cu") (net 4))
 (segment (start 59.3544 44.4954) (end 55.2364 44.4954) (width 0.4) (layer "F.Cu") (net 4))
 (segment (start 52.5334 36.4044) (end 52.5334 34.3724) (width 0.4) (layer "F.Cu") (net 4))
 (segment (start 25.3449 46.0744) (end 25.3449 35.5069) (width 0.4) (layer "F.Cu") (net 4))
 (segment (start 37.0394 57.4864) (end 37.3254 57.7724) (width 0.4) (layer "F.Cu") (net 4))
 (segment (start 35.7694 56.4704) (end 21.6724 56.4704) (width 0.4) (layer "F.Cu") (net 4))
 (segment (start 51.776 33.615) (end 51.776 30.812) (width 0.4) (layer "F.Cu") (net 4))
 (segment (start 55.2364 44.4954) (end 54.1834 45.5484) (width 0.4) (layer "F.Cu") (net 4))
 (segment (start 37.3254 57.7724) (end 46.8474 57.7724) (width 0.4) (layer "F.Cu") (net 4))
 (segment (start 36.7854 57.4864) (end 37.0394 57.4864) (width 0.4) (layer "F.Cu") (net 4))
 (segment (start 22.0354 46.0744) (end 25.3449 46.0744) (width 0.4) (layer "F.Cu") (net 4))
 (segment (start 52.7874 45.5484) (end 50.976 43.737) (width 0.4) (layer "F.Cu") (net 4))
 (segment (start 51.5174 37.4204) (end 52.5334 36.4044) (width 0.4) (layer "F.Cu") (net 4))
 (segment (start 25.3449 35.5069) (end 25.1248 35.2868) (width 0.4) (layer "F.Cu") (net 4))
 (segment (start 19.558 48.5518) (end 22.0354 46.0744) (width 0.4) (layer "F.Cu") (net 4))
 (segment (start 36.7854 57.4864) (end 35.7694 56.4704) (width 0.4) (layer "F.Cu") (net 4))
 (segment (start 52.0254 37.4204) (end 52.576 37.971) (width 0.4) (layer "F.Cu") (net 4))
 (segment (start 19.558 54.356) (end 19.558 48.5518) (width 0.4) (layer "F.Cu") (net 4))
 (segment (start 51.5174 37.4204) (end 52.0254 37.4204) (width 0.4) (layer "F.Cu") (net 4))
 (via (at 59.3914 44.5324) (size 2.6) (drill 1.6) (layers "F.Cu" "B.Cu") (free yes) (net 4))
 (via (at 31.9594 60.0264) (size 2.6) (drill 1.6) (layers "F.Cu" "B.Cu") (free yes) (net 4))
 (segment (start 31.9594 60.0264) (end 43.8974 60.0264) (width 0.4) (layer "B.Cu") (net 4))
 (segment (start 43.8974 60.0264) (end 59.3914 44.5324) (width 0.4) (layer "B.Cu") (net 4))
 (segment (start 58.1214 66.3764) (end 58.1214 55.7084) (width 0.4) (layer "F.Cu") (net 5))
 (segment (start 50.7554 35.3884) (end 49.9934 36.1504) (width 0.4) (layer "F.Cu") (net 5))
 (segment (start 56.5974 54.1844) (end 49.4854 54.1844) (width 0.4) (layer "F.Cu") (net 5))
 (segment (start 50.8334 35.3884) (end 50.7554 35.3884) (width 0.4) (layer "F.Cu") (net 5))
 (segment (start 50.5014 73.9964) (end 58.1214 66.3764) (width 0.4) (layer "F.Cu") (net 5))
 (segment (start 34.7534 71.9644) (end 36.7854 73.9964) (width 0.4) (layer "F.Cu") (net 5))
 (segment (start 46.4374 47.8344) (end 46.4374 51.1364) (width 0.4) (layer "F.Cu") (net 5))
 (segment (start 48.0376 36.1504) (end 48.006 36.182) (width 0.4) (layer "F.Cu") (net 5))
 (segment (start 46.4374 51.1364) (end 49.4854 54.1844) (width 0.4) (layer "F.Cu") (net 5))
 (segment (start 36.7854 73.9964) (end 50.5014 73.9964) (width 0.4) (layer "F.Cu") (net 5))
 (segment (start 36.7854 67.6464) (end 34.7534 69.6784) (width 0.4) (layer "F.Cu") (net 5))
 (segment (start 58.1214 55.7084) (end 56.5974 54.1844) (width 0.4) (layer "F.Cu") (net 5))
 (segment (start 49.9934 36.1504) (end 48.0376 36.1504) (width 0.4) (layer "F.Cu") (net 5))
 (segment (start 34.7534 69.6784) (end 34.7534 71.9644) (width 0.4) (layer "F.Cu") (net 5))
 (via (at 50.8334 35.3884) (size 2.6) (drill 1.6) (layers "F.Cu" "B.Cu") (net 5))
 (via (at 46.4374 47.8344) (size 2.6) (drill 1.6) (layers "F.Cu" "B.Cu") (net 5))
 (segment (start 50.8334 35.3884) (end 50.7554 35.3884) (width 0.4) (layer "B.Cu") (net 5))
 (segment (start 50.7554 35.3884) (end 46.4374 39.7064) (width 0.4) (layer "B.Cu") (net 5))
 (segment (start 46.4374 39.7064) (end 46.4374 47.8344) (width 0.4) (layer "B.Cu") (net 5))
 (segment (start 47.9364 36.9124) (end 48.006 36.982) (width 0.4) (layer "F.Cu") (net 6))
 (segment (start 35.2614 63.5824) (end 35.2614 62.0584) (width 0.4) (layer "F.Cu") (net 6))
 (segment (start 43.3894 38.1824) (end 44.5898 36.982) (width 0.4) (layer "F.Cu") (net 6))
 (segment (start 56.5974 56.9784) (end 55.3274 55.7084) (width 0.4) (layer "F.Cu") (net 6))
 (segment (start 45.6754 55.7084) (end 43.3894 53.4224) (width 0.4) (layer "F.Cu") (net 6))
 (segment (start 35.2614 62.0584) (end 36.0234 61.2964) (width 0.4) (layer "F.Cu") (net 6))
 (segment (start 44.5898 36.982) (end 48.006 36.982) (width 0.4) (layer "F.Cu") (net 6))
 (segment (start 56.5974 59.5184) (end 56.5974 56.9784) (width 0.4) (layer "F.Cu") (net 6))
 (segment (start 55.8354 60.2804) (end 56.5974 59.5184) (width 0.4) (layer "F.Cu") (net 6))
 (segment (start 44.9134 60.2804) (end 55.8354 60.2804) (width 0.4) (layer "F.Cu") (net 6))
 (segment (start 43.3894 53.4224) (end 43.3894 38.1824) (width 0.4) (layer "F.Cu") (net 6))
 (segment (start 43.8974 61.2964) (end 44.9134 60.2804) (width 0.4) (layer "F.Cu") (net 6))
 (segment (start 36.0234 61.2964) (end 43.8974 61.2964) (width 0.4) (layer "F.Cu") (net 6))
 (segment (start 36.7854 65.1064) (end 35.2614 63.5824) (width 0.4) (layer "F.Cu") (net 6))
 (segment (start 55.3274 55.7084) (end 45.6754 55.7084) (width 0.4) (layer "F.Cu") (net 6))
 (segment (start 54.3114 43.7704) (end 54.3114 42.664916) (width 0.4) (layer "F.Cu") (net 8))
 (segment (start 54.3114 42.664916) (end 54.176 42.529516) (width 0.4) (layer "F.Cu") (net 8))
 (segment (start 54.176 42.529516) (end 54.176 39.152) (width 0.4) (layer "F.Cu") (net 8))
 (segment (start 53.3864 44.4954) (end 53.5864 44.4954) (width 0.4) (layer "F.Cu") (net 8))
 (segment (start 53.5864 44.4954) (end 54.3114 43.7704) (width 0.4) (layer "F.Cu") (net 8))
 (segment (start 54.976 41.133) (end 55.2364 41.3934) (width 0.4) (layer "F.Cu") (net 9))
 (segment (start 55.2364 41.3934) (end 55.2364 43.0454) (width 0.4) (layer "F.Cu") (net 9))
 (segment (start 54.976 39.152) (end 54.976 41.133) (width 0.4) (layer "F.Cu") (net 9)))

